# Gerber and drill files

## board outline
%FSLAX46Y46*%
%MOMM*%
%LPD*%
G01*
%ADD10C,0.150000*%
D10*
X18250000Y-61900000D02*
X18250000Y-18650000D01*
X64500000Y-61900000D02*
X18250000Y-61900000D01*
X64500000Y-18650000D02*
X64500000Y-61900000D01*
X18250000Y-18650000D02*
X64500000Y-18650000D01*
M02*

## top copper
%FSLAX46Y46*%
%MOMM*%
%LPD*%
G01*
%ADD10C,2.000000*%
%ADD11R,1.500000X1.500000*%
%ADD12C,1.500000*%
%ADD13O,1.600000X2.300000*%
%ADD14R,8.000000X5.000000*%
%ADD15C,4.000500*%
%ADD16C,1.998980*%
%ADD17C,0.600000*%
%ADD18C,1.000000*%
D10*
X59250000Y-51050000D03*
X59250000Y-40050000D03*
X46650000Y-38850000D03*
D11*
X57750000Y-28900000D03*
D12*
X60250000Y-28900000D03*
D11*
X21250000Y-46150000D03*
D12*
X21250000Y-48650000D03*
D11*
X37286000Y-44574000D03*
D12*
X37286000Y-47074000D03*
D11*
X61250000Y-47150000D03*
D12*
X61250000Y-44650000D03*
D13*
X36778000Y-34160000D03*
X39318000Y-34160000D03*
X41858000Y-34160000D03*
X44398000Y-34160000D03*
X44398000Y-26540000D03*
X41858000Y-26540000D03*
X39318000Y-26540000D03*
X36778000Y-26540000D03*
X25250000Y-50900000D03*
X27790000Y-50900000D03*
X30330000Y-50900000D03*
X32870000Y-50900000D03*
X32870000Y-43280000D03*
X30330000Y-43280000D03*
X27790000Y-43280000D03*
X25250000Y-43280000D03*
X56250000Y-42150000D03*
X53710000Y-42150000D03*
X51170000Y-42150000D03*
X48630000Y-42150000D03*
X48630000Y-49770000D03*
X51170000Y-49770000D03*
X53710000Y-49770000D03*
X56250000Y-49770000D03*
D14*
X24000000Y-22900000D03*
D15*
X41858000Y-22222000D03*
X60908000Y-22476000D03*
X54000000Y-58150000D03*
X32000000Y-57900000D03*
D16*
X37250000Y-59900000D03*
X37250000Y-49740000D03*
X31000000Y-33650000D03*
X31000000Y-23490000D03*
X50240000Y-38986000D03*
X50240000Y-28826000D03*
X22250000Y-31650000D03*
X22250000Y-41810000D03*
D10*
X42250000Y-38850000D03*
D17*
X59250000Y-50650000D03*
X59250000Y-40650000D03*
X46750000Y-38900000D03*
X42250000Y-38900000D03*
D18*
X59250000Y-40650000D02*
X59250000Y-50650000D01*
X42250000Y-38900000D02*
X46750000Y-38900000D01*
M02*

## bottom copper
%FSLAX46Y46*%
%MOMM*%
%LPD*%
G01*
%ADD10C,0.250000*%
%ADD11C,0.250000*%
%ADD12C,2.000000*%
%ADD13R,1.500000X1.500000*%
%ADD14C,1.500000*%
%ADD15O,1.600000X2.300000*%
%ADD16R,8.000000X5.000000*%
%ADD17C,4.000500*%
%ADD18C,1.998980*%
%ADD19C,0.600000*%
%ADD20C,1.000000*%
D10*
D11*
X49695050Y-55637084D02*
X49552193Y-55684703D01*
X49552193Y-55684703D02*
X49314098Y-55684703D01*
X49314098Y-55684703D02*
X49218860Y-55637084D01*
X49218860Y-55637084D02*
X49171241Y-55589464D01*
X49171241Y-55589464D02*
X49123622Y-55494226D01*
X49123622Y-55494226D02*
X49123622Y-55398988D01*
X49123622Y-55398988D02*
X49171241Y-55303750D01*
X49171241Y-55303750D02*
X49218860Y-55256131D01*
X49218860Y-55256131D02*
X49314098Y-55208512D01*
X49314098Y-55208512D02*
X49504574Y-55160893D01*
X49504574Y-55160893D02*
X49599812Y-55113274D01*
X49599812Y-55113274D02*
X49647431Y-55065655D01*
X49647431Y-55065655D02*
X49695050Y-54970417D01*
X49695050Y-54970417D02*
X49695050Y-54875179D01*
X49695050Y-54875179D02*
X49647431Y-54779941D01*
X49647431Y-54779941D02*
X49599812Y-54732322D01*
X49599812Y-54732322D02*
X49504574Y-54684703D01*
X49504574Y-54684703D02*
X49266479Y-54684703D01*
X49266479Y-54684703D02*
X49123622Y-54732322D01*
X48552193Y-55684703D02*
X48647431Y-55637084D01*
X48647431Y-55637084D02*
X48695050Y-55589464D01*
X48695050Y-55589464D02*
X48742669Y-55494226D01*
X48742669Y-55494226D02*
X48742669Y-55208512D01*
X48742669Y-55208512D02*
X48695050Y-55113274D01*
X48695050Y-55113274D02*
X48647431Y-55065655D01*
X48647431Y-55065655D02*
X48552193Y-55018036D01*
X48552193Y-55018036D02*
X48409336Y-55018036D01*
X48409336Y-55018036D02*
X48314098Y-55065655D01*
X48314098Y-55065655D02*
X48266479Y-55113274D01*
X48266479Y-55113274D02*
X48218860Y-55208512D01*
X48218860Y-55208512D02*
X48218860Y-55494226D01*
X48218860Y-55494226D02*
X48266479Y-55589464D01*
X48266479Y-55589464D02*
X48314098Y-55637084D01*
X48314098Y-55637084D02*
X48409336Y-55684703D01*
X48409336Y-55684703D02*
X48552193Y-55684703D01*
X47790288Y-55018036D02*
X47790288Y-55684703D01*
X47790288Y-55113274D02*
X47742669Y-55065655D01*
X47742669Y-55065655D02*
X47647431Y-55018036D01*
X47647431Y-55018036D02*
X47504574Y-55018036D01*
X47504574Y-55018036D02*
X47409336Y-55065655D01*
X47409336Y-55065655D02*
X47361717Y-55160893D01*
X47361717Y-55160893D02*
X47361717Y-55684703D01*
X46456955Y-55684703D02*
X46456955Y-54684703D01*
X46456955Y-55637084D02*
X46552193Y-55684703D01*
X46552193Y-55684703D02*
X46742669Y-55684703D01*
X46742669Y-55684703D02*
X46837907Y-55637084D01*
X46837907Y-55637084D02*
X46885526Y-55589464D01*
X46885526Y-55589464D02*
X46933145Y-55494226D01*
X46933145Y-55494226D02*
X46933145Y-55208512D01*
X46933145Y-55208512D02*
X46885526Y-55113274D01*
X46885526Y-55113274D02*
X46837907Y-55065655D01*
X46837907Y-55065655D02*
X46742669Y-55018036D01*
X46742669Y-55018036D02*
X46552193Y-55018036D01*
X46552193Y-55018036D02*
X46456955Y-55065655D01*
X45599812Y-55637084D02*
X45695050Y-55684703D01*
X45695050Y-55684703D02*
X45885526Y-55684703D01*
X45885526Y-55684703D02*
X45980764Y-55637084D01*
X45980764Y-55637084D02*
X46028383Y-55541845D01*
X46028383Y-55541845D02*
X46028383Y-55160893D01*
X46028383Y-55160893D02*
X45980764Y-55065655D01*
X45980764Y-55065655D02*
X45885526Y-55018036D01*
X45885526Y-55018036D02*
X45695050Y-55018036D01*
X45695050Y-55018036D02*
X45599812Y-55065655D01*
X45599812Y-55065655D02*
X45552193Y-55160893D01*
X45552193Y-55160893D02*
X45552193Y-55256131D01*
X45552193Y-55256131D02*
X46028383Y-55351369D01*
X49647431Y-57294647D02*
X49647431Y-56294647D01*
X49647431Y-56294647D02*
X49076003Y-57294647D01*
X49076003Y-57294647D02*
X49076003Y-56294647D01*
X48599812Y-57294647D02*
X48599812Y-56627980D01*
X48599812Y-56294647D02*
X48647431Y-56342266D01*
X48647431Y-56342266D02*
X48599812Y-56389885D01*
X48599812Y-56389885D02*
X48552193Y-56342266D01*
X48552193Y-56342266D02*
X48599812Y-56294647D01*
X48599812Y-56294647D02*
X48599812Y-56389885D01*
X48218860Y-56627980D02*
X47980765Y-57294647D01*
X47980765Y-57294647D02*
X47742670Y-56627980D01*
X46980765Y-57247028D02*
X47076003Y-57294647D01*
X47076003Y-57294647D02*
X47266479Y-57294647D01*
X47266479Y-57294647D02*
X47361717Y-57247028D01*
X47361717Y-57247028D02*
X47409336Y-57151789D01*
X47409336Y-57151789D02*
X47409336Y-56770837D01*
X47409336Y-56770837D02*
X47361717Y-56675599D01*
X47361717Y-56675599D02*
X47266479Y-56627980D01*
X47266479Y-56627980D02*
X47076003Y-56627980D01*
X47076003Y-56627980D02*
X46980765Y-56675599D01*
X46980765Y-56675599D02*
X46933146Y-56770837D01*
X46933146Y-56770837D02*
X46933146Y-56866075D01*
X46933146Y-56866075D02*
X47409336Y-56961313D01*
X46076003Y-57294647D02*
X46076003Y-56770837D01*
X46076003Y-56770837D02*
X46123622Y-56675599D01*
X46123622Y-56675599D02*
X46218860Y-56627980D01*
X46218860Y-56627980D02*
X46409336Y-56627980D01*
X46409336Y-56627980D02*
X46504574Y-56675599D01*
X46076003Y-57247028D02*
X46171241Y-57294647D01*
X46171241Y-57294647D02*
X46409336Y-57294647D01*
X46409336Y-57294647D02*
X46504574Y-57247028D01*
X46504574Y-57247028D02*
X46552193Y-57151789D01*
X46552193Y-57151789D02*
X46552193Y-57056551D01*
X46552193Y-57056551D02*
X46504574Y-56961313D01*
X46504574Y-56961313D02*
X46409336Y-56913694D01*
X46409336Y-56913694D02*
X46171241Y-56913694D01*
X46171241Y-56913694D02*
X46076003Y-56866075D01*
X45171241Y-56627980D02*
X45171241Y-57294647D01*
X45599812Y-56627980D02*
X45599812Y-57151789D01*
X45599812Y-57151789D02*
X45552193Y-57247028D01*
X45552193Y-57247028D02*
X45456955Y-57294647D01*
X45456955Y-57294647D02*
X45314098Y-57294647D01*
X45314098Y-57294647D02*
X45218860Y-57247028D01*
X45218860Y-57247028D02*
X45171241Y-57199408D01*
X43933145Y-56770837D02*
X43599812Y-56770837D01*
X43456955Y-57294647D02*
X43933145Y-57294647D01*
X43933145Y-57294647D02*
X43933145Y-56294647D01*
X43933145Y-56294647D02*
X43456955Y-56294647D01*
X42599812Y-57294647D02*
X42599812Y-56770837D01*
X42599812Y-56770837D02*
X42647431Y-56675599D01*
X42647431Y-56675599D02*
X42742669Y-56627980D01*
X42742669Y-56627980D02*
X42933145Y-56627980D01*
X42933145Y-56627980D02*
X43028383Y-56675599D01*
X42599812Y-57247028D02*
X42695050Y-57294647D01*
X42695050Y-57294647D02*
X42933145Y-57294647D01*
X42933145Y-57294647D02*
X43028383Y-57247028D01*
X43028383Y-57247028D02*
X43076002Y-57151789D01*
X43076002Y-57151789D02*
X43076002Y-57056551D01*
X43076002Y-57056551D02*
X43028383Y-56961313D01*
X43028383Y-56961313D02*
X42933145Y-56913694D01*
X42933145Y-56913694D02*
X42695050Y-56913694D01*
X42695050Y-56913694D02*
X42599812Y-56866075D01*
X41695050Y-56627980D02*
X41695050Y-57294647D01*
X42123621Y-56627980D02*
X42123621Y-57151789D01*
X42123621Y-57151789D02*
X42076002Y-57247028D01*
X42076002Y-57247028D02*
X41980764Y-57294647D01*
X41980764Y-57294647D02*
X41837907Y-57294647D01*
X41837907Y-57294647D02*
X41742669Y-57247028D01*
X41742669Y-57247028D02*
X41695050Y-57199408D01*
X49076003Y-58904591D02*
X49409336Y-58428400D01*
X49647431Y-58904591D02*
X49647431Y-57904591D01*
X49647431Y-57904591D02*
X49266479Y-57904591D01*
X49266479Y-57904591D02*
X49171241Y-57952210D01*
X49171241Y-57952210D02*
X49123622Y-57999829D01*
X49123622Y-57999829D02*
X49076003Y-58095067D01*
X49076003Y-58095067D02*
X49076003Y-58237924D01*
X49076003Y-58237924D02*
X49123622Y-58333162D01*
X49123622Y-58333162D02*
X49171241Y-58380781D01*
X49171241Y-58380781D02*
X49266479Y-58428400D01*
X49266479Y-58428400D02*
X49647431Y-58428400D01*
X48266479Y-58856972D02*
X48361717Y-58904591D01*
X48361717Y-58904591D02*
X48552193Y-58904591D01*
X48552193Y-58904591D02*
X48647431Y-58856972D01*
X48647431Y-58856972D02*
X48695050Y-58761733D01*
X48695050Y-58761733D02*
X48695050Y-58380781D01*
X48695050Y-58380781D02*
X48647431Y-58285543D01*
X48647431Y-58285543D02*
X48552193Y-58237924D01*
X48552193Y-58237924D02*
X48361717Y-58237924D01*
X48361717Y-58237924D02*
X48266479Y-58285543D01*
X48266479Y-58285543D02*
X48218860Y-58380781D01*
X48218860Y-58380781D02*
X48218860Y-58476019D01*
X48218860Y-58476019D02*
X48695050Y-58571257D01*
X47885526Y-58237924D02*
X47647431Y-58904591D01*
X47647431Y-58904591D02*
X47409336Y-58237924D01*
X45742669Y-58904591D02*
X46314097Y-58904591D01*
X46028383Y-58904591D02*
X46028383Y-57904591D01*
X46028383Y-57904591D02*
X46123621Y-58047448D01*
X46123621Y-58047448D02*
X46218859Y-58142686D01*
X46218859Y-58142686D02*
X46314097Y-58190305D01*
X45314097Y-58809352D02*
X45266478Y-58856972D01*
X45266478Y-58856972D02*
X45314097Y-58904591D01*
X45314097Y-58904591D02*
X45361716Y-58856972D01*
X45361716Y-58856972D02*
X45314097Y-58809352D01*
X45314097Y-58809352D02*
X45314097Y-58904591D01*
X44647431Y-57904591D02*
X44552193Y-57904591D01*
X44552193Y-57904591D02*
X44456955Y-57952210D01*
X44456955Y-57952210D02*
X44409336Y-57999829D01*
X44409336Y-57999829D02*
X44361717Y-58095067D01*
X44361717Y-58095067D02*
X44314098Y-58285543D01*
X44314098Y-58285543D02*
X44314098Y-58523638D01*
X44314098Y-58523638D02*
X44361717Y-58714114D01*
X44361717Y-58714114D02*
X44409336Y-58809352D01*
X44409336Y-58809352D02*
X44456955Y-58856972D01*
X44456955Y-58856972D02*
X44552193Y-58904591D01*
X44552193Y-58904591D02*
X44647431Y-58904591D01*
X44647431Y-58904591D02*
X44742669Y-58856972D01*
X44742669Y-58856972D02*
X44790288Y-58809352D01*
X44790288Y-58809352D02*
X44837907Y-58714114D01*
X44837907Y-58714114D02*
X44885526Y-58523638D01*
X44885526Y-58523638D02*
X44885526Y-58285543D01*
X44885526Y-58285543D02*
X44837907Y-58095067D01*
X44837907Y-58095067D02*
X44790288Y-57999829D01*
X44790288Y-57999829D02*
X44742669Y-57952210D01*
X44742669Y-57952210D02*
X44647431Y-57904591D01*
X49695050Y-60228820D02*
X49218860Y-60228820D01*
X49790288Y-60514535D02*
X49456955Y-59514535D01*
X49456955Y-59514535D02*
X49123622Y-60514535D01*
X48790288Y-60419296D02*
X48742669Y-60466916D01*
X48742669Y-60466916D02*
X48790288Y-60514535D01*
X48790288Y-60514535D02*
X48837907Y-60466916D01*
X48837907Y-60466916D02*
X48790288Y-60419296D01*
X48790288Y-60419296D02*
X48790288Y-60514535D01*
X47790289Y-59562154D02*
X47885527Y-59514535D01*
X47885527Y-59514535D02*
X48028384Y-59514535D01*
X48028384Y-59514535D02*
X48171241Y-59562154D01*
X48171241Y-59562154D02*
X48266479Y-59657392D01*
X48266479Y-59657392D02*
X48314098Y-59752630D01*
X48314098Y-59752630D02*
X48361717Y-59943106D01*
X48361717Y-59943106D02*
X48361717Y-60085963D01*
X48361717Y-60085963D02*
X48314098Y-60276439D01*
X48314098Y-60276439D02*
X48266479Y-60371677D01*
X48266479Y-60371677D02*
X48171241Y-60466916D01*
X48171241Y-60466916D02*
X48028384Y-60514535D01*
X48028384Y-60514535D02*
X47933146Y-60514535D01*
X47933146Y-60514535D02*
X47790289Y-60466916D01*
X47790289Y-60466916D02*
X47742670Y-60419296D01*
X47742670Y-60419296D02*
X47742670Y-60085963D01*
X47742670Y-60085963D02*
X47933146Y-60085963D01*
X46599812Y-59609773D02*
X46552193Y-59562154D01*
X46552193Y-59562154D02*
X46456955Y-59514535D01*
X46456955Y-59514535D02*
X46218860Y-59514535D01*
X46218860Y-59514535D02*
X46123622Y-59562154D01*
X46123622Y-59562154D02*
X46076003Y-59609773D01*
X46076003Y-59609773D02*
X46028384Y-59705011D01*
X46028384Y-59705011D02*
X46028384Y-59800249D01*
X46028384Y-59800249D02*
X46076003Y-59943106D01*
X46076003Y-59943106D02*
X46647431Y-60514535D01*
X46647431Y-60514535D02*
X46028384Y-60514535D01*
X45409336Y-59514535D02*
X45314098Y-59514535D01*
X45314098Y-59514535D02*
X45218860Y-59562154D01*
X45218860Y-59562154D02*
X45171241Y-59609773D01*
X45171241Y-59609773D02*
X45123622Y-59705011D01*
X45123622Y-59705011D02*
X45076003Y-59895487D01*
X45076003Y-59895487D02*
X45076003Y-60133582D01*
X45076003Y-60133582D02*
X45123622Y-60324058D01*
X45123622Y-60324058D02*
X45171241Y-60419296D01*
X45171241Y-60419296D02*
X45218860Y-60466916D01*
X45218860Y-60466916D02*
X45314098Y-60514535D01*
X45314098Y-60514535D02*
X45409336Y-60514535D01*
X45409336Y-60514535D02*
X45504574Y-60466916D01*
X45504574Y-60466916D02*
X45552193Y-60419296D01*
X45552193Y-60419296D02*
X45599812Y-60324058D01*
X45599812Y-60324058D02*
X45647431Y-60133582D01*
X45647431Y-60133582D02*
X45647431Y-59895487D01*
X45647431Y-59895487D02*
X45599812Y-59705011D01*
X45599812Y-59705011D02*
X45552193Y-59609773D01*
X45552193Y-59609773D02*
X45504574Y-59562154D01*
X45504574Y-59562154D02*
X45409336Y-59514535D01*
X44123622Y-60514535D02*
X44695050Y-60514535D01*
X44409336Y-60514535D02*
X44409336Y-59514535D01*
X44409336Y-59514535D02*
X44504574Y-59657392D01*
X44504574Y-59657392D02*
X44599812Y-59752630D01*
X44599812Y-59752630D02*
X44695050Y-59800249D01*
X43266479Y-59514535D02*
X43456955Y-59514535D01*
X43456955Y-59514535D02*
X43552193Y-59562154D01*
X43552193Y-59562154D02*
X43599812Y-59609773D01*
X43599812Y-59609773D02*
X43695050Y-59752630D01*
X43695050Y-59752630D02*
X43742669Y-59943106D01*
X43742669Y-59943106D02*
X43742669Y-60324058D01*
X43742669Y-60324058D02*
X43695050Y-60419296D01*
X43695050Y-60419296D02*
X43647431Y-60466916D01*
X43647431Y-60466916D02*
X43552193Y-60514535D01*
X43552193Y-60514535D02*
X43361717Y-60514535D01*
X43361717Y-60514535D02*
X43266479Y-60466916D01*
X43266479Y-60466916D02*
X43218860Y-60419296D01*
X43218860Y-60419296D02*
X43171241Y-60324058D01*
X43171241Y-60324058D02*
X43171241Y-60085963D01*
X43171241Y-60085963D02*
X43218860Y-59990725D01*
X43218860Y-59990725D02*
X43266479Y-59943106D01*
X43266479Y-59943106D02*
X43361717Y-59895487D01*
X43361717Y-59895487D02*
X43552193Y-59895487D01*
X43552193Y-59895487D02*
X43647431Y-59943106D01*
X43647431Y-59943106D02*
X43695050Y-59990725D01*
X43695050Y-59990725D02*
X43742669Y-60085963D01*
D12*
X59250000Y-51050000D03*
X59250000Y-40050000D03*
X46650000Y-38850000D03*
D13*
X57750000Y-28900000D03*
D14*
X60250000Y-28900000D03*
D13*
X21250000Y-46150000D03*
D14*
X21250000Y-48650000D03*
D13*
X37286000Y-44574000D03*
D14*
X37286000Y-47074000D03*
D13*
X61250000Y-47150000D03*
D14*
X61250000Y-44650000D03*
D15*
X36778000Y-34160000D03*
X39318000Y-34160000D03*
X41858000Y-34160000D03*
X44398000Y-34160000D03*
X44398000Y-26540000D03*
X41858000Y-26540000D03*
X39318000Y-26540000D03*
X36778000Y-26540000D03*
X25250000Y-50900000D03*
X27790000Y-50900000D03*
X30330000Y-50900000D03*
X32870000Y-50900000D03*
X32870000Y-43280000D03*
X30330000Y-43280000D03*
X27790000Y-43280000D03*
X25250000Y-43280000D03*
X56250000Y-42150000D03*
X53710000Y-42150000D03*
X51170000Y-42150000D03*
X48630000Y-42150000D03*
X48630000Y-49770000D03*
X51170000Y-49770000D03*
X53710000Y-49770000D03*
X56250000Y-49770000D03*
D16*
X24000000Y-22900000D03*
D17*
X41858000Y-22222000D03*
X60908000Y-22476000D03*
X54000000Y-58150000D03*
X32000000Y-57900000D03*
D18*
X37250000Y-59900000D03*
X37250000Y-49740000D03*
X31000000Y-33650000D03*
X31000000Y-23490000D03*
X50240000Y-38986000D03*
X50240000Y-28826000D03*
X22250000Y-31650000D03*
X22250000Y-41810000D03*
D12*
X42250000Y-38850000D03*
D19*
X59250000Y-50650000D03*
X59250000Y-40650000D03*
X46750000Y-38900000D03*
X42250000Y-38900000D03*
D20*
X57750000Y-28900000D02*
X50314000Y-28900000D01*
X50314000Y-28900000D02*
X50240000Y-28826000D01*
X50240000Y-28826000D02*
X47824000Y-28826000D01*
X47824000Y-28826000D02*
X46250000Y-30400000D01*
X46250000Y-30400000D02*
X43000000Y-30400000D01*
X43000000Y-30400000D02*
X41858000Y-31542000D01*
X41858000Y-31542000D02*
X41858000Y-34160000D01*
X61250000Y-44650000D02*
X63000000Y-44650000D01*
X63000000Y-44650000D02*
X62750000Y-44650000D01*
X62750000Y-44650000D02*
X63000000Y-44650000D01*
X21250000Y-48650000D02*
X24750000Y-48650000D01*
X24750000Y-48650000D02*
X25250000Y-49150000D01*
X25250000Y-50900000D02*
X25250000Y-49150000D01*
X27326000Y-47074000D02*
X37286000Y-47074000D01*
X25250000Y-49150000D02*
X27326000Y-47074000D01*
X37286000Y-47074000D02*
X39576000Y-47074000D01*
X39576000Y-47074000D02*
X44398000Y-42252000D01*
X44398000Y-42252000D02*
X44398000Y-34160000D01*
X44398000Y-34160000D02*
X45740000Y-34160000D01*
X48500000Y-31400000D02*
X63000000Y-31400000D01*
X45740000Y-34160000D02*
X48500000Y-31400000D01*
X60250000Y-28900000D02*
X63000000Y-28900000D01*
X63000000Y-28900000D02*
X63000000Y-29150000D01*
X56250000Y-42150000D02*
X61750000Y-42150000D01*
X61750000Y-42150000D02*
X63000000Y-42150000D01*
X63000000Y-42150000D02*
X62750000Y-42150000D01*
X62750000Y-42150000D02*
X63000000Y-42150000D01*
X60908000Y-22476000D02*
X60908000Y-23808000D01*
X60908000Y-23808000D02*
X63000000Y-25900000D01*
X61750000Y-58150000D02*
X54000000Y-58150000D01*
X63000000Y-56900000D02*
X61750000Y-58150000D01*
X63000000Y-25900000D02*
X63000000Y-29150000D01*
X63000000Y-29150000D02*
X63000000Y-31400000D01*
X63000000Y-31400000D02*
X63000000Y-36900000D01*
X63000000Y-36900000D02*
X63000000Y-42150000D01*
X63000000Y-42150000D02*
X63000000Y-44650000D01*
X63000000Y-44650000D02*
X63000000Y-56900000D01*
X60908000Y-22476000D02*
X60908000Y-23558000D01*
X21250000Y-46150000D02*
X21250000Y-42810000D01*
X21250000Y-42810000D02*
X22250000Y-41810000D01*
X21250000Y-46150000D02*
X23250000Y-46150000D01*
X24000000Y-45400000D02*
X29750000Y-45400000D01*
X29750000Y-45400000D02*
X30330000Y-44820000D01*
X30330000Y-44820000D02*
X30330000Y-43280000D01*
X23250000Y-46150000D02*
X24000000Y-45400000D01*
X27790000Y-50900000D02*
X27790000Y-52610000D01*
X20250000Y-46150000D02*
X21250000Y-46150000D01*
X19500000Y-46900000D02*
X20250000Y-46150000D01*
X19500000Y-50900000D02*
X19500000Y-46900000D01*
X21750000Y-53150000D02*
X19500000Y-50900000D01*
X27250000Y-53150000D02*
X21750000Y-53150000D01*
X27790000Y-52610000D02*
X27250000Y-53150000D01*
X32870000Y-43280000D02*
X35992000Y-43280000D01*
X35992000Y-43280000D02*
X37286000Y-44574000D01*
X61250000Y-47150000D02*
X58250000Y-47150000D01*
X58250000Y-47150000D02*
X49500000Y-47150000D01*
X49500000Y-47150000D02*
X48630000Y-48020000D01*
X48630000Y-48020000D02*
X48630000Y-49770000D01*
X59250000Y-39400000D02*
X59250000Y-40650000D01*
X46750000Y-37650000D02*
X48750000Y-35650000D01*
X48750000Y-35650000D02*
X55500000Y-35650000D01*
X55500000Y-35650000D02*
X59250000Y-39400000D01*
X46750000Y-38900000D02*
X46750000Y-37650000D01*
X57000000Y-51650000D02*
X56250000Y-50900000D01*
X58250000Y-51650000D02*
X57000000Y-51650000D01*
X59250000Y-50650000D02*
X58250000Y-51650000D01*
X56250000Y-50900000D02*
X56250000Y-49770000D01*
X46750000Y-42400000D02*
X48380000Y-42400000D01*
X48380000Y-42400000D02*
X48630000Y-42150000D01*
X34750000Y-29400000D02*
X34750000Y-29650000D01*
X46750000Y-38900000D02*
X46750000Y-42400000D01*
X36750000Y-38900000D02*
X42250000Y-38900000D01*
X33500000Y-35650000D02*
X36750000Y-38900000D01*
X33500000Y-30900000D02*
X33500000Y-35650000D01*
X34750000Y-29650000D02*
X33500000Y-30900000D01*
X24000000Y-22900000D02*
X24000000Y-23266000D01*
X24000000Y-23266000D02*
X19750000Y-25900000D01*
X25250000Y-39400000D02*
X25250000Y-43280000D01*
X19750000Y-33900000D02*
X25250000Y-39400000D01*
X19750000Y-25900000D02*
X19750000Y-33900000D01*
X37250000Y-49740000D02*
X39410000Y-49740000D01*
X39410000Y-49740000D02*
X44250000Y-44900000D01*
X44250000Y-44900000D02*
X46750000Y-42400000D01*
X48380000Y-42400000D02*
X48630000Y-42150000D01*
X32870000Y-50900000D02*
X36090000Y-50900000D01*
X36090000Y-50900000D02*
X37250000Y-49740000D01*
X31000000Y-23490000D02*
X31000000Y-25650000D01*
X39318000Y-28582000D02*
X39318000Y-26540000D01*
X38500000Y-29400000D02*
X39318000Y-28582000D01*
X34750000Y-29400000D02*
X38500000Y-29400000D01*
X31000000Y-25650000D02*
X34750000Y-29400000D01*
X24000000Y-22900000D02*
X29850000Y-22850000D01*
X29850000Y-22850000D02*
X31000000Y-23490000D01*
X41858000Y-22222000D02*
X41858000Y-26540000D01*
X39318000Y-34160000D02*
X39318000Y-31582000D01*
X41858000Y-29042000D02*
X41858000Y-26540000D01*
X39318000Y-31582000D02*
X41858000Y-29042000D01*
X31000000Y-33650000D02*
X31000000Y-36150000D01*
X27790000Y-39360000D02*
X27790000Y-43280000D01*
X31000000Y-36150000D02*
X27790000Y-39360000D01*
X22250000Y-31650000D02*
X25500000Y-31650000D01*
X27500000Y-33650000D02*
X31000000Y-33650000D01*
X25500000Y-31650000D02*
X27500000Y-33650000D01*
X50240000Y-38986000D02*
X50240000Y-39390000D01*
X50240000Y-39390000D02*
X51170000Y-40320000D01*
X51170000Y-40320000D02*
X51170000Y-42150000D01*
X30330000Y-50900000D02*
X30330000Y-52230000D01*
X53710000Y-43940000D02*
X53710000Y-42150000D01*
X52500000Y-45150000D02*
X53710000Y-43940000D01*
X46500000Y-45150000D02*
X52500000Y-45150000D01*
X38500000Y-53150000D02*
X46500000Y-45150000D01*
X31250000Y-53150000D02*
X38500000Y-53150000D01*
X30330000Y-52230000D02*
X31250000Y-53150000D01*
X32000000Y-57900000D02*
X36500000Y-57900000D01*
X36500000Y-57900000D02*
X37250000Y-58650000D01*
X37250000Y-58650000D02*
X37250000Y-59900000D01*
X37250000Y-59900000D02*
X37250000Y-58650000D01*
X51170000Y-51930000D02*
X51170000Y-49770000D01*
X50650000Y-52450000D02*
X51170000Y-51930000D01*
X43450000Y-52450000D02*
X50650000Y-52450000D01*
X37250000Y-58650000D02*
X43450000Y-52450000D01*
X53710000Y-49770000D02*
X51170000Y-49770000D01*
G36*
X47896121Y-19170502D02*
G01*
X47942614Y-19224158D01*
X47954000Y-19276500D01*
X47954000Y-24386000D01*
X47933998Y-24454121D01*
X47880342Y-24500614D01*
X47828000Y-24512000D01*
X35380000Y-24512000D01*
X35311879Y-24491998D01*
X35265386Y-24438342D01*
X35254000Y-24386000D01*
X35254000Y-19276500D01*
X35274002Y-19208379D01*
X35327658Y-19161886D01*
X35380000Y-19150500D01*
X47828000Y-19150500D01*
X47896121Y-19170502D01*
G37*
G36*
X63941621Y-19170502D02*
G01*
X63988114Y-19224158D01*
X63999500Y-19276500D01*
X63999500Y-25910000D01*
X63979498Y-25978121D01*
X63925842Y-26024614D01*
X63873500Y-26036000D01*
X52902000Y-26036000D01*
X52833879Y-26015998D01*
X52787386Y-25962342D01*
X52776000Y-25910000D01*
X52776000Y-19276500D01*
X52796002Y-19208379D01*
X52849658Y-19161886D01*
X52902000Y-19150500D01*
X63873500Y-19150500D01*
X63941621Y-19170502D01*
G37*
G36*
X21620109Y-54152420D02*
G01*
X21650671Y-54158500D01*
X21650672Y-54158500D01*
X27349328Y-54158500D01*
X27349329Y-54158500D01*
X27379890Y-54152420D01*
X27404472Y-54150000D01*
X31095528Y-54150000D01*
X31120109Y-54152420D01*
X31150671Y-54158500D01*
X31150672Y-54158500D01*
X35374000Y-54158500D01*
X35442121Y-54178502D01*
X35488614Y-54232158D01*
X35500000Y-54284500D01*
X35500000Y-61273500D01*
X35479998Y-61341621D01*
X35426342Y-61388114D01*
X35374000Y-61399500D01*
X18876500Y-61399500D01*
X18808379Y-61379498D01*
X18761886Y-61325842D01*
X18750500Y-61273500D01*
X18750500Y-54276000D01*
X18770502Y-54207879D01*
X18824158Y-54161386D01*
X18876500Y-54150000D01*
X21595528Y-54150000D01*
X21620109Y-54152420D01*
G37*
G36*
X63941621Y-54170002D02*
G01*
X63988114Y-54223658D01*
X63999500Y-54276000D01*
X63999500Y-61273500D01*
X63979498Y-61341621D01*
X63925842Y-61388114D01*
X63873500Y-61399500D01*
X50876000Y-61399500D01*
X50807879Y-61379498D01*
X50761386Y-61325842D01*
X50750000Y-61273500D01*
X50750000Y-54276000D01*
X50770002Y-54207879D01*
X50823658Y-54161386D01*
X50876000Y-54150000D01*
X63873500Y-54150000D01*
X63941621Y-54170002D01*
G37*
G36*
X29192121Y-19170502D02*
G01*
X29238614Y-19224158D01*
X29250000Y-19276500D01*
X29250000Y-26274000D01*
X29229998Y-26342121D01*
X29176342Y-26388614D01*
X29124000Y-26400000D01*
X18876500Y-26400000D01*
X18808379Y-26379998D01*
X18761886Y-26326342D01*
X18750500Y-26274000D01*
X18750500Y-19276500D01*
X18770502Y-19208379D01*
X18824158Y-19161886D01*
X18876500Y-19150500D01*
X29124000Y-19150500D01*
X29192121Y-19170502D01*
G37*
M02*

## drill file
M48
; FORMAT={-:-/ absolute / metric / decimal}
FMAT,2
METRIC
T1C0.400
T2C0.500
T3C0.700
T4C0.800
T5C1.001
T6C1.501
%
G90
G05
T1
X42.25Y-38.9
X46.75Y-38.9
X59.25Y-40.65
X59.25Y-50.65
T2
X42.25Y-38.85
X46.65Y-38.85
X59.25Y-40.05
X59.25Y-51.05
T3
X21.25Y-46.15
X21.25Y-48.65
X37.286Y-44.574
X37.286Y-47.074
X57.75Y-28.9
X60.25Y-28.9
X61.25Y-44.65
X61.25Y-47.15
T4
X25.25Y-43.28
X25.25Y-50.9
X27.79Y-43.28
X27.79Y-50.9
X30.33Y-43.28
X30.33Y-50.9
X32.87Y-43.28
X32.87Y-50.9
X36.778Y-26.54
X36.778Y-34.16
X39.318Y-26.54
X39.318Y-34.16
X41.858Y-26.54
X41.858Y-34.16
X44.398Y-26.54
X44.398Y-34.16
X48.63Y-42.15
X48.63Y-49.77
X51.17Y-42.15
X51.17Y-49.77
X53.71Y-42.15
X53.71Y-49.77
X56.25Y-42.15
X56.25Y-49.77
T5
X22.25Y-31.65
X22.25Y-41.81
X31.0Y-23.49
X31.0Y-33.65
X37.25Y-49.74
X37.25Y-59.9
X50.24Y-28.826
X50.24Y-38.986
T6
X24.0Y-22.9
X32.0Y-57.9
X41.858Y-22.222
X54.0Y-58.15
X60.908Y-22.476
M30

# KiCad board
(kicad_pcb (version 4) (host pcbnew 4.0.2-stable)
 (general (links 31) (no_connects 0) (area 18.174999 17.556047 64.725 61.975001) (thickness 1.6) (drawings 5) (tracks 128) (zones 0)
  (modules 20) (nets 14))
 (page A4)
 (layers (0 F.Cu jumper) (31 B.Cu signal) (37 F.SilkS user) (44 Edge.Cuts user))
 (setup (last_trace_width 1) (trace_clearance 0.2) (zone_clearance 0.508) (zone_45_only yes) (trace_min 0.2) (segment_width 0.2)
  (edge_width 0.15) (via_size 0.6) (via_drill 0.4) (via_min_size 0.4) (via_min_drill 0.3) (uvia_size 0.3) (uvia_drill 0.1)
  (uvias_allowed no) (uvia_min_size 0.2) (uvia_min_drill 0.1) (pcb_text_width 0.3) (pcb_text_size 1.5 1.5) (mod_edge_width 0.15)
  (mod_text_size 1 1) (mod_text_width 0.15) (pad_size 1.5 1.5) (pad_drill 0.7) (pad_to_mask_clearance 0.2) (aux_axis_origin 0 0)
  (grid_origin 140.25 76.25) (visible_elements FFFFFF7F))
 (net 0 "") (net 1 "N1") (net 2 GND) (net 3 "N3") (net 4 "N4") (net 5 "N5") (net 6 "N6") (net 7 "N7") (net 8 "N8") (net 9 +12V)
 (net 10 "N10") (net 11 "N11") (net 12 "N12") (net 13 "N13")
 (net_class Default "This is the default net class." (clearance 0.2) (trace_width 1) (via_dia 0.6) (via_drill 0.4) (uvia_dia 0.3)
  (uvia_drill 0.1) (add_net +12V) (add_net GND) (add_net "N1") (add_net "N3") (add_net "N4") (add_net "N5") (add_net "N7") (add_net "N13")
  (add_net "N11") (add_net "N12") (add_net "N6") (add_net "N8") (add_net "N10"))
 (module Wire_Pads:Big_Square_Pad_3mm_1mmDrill (layer F.Cu) (at 59.25 51.05)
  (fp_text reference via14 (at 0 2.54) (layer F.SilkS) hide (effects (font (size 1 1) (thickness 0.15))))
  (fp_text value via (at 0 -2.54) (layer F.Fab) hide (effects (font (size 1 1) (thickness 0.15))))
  (pad 1 thru_hole circle (at 0 0) (size 2 2) (drill 0.5) (layers *.Cu *.Mask F.SilkS)))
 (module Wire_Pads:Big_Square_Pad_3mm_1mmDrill (layer F.Cu) (at 59.25 40.05)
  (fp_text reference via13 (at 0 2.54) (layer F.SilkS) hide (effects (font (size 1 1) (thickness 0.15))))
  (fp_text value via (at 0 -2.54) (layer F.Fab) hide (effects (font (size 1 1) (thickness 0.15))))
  (pad 1 thru_hole circle (at 0 0) (size 2 2) (drill 0.5) (layers *.Cu *.Mask F.SilkS)))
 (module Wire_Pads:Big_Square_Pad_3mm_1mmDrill (layer F.Cu) (at 46.65 38.85)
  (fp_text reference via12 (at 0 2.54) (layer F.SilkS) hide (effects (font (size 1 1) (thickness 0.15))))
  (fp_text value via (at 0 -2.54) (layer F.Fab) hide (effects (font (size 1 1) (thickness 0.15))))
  (pad 1 thru_hole circle (at 0 0) (size 2 2) (drill 0.5) (layers *.Cu *.Mask F.SilkS)))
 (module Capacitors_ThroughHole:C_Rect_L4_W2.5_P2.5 (layer F.Cu) (at 57.75 28.9)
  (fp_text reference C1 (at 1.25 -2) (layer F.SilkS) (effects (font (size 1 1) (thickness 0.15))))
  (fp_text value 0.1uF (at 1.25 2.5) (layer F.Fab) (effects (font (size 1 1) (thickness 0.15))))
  (pad 1 thru_hole rect (at 0 0) (size 1.5 1.5) (drill 0.7) (layers *.Cu *.Mask F.SilkS) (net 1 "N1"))
  (pad 2 thru_hole circle (at 2.5 0) (size 1.5 1.5) (drill 0.7) (layers *.Cu *.Mask F.SilkS) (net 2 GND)))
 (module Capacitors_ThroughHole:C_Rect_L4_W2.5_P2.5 (layer F.Cu) (at 21.25 46.15 270)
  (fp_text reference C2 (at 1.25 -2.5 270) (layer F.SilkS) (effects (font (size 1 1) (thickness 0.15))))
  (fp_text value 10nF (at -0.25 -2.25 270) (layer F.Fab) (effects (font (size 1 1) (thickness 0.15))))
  (pad 1 thru_hole rect (at 0 0 270) (size 1.5 1.5) (drill 0.7) (layers *.Cu *.Mask F.SilkS) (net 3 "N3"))
  (pad 2 thru_hole circle (at 2.5 0 270) (size 1.5 1.5) (drill 0.7) (layers *.Cu *.Mask F.SilkS) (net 2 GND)))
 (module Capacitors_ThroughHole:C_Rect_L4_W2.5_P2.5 (layer F.Cu) (at 37.286 44.574 270)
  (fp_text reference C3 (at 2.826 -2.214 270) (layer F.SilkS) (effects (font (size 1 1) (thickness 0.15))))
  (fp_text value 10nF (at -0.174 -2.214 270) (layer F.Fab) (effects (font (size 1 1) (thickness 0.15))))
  (pad 1 thru_hole rect (at 0 0 270) (size 1.5 1.5) (drill 0.7) (layers *.Cu *.Mask F.SilkS) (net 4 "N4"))
  (pad 2 thru_hole circle (at 2.5 0 270) (size 1.5 1.5) (drill 0.7) (layers *.Cu *.Mask F.SilkS) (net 2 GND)))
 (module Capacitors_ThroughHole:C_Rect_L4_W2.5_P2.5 (layer F.Cu) (at 61.25 47.15 90)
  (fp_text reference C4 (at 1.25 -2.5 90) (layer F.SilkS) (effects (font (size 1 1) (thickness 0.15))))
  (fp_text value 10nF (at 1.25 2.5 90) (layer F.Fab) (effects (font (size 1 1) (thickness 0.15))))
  (pad 1 thru_hole rect (at 0 0 90) (size 1.5 1.5) (drill 0.7) (layers *.Cu *.Mask F.SilkS) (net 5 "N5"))
  (pad 2 thru_hole circle (at 2.5 0 90) (size 1.5 1.5) (drill 0.7) (layers *.Cu *.Mask F.SilkS) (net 2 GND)))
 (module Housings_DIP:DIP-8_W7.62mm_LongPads (layer F.Cu) (at 36.778 34.16 90)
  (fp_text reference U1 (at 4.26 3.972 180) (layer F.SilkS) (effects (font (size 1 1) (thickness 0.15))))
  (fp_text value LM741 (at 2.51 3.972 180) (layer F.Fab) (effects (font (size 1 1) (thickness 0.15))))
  (pad 1 thru_hole oval (at 0 0 90) (size 2.3 1.6) (drill 0.8) (layers *.Cu *.Mask F.SilkS) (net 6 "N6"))
  (pad 2 thru_hole oval (at 0 2.54 90) (size 2.3 1.6) (drill 0.8) (layers *.Cu *.Mask F.SilkS) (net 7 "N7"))
  (pad 3 thru_hole oval (at 0 5.08 90) (size 2.3 1.6) (drill 0.8) (layers *.Cu *.Mask F.SilkS) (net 1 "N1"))
  (pad 4 thru_hole oval (at 0 7.62 90) (size 2.3 1.6) (drill 0.8) (layers *.Cu *.Mask F.SilkS) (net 2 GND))
  (pad 5 thru_hole oval (at 7.62 7.62 90) (size 2.3 1.6) (drill 0.8) (layers *.Cu *.Mask F.SilkS) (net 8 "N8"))
  (pad 6 thru_hole oval (at 7.62 5.08 90) (size 2.3 1.6) (drill 0.8) (layers *.Cu *.Mask F.SilkS) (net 7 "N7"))
  (pad 7 thru_hole oval (at 7.62 2.54 90) (size 2.3 1.6) (drill 0.8) (layers *.Cu *.Mask F.SilkS) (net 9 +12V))
  (pad 8 thru_hole oval (at 7.62 0 90) (size 2.3 1.6) (drill 0.8) (layers *.Cu *.Mask F.SilkS)))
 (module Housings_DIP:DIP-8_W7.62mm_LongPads (layer F.Cu) (at 25.25 50.9 90)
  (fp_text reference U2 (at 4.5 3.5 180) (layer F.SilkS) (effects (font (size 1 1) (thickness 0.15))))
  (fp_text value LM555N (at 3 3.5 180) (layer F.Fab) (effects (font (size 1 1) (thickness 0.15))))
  (pad 1 thru_hole oval (at 0 0 90) (size 2.3 1.6) (drill 0.8) (layers *.Cu *.Mask F.SilkS) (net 2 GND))
  (pad 2 thru_hole oval (at 0 2.54 90) (size 2.3 1.6) (drill 0.8) (layers *.Cu *.Mask F.SilkS) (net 3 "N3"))
  (pad 3 thru_hole oval (at 0 5.08 90) (size 2.3 1.6) (drill 0.8) (layers *.Cu *.Mask F.SilkS) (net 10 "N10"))
  (pad 4 thru_hole oval (at 0 7.62 90) (size 2.3 1.6) (drill 0.8) (layers *.Cu *.Mask F.SilkS) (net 9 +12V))
  (pad 5 thru_hole oval (at 7.62 7.62 90) (size 2.3 1.6) (drill 0.8) (layers *.Cu *.Mask F.SilkS) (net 4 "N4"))
  (pad 6 thru_hole oval (at 7.62 5.08 90) (size 2.3 1.6) (drill 0.8) (layers *.Cu *.Mask F.SilkS) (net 3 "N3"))
  (pad 7 thru_hole oval (at 7.62 2.54 90) (size 2.3 1.6) (drill 0.8) (layers *.Cu *.Mask F.SilkS) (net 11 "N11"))
  (pad 8 thru_hole oval (at 7.62 0 90) (size 2.3 1.6) (drill 0.8) (layers *.Cu *.Mask F.SilkS) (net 9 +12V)))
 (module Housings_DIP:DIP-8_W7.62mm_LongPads (layer F.Cu) (at 56.25 42.15 270)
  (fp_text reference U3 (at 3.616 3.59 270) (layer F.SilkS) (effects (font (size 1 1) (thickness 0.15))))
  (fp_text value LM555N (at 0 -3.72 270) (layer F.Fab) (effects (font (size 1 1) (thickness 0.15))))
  (pad 1 thru_hole oval (at 0 0 270) (size 2.3 1.6) (drill 0.8) (layers *.Cu *.Mask F.SilkS) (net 2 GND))
  (pad 2 thru_hole oval (at 0 2.54 270) (size 2.3 1.6) (drill 0.8) (layers *.Cu *.Mask F.SilkS) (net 10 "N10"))
  (pad 3 thru_hole oval (at 0 5.08 270) (size 2.3 1.6) (drill 0.8) (layers *.Cu *.Mask F.SilkS) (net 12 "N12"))
  (pad 4 thru_hole oval (at 0 7.62 270) (size 2.3 1.6) (drill 0.8) (layers *.Cu *.Mask F.SilkS) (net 9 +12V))
  (pad 5 thru_hole oval (at 7.62 7.62 270) (size 2.3 1.6) (drill 0.8) (layers *.Cu *.Mask F.SilkS) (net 5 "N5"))
  (pad 6 thru_hole oval (at 7.62 5.08 270) (size 2.3 1.6) (drill 0.8) (layers *.Cu *.Mask F.SilkS) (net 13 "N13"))
  (pad 7 thru_hole oval (at 7.62 2.54 270) (size 2.3 1.6) (drill 0.8) (layers *.Cu *.Mask F.SilkS) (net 13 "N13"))
  (pad 8 thru_hole oval (at 7.62 0 270) (size 2.3 1.6) (drill 0.8) (layers *.Cu *.Mask F.SilkS) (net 9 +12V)))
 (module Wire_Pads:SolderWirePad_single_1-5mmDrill (layer F.Cu) (at 24 22.9 180)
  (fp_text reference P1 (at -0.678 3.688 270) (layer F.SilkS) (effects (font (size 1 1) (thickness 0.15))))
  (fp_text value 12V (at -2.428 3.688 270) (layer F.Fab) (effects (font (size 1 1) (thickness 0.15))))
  (pad 1 thru_hole rect (at 0 0 180) (size 8 5) (drill 1.50114) (layers *.Cu *.Mask F.SilkS) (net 9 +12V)))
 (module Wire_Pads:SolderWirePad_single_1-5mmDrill (layer F.Cu) (at 41.858 22.222 270)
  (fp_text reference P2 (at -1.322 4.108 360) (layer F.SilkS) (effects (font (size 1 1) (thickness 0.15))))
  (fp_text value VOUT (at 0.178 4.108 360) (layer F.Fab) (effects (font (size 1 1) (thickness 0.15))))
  (pad 1 thru_hole circle (at 0 0 270) (size 4.0005 4.0005) (drill 1.50114) (layers *.Cu *.Mask F.SilkS) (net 7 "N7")))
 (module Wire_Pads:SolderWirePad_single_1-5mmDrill (layer F.Cu) (at 60.908 22.476)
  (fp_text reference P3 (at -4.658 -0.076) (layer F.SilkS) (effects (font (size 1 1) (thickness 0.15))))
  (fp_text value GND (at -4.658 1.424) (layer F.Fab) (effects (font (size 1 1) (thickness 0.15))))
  (pad 1 thru_hole circle (at 0 0) (size 4.0005 4.0005) (drill 1.50114) (layers *.Cu *.Mask F.SilkS) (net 2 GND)))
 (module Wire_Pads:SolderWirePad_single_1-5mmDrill (layer F.Cu) (at 54 58.15)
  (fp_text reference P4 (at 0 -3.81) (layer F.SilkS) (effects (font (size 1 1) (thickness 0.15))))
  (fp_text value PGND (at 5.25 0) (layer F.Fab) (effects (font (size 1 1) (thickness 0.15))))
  (pad 1 thru_hole circle (at 0 0) (size 4.0005 4.0005) (drill 1.50114) (layers *.Cu *.Mask F.SilkS) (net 2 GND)))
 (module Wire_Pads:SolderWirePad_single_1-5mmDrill (layer F.Cu) (at 32 57.9)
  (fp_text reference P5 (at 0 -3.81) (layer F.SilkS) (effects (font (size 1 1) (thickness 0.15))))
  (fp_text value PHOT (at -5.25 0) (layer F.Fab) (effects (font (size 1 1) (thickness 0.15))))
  (pad 1 thru_hole circle (at 0 0) (size 4.0005 4.0005) (drill 1.50114) (layers *.Cu *.Mask F.SilkS) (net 13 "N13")))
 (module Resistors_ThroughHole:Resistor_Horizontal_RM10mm (layer F.Cu) (at 37.25 59.9 90)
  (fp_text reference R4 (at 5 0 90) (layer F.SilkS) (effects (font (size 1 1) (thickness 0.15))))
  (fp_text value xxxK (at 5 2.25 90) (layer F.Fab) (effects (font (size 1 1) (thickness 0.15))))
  (pad 1 thru_hole circle (at 0 0 90) (size 1.99898 1.99898) (drill 1.00076) (layers *.Cu *.SilkS *.Mask) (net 13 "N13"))
  (pad 2 thru_hole circle (at 10.16 0 90) (size 1.99898 1.99898) (drill 1.00076) (layers *.Cu *.SilkS *.Mask) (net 9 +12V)))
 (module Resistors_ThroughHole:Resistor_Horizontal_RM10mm (layer F.Cu) (at 31 33.65 90)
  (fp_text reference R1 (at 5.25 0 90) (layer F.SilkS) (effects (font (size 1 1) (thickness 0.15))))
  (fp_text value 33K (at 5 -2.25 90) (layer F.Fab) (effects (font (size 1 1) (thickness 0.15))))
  (pad 1 thru_hole circle (at 0 0 90) (size 1.99898 1.99898) (drill 1.00076) (layers *.Cu *.SilkS *.Mask) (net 11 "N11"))
  (pad 2 thru_hole circle (at 10.16 0 90) (size 1.99898 1.99898) (drill 1.00076) (layers *.Cu *.SilkS *.Mask) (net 9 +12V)))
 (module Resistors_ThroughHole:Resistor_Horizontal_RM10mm (layer F.Cu) (at 50.24 38.986 90)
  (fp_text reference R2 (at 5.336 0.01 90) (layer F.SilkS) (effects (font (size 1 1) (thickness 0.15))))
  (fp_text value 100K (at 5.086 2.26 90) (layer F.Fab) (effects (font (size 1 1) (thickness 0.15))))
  (pad 1 thru_hole circle (at 0 0 90) (size 1.99898 1.99898) (drill 1.00076) (layers *.Cu *.SilkS *.Mask) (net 12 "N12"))
  (pad 2 thru_hole circle (at 10.16 0 90) (size 1.99898 1.99898) (drill 1.00076) (layers *.Cu *.SilkS *.Mask) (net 1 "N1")))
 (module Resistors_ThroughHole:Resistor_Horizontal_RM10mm (layer F.Cu) (at 22.25 31.65 270)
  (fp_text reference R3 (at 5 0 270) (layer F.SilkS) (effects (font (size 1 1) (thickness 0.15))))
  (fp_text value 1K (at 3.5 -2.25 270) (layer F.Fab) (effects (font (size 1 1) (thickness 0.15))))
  (pad 1 thru_hole circle (at 0 0 270) (size 1.99898 1.99898) (drill 1.00076) (layers *.Cu *.SilkS *.Mask) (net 11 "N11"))
  (pad 2 thru_hole circle (at 10.16 0 270) (size 1.99898 1.99898) (drill 1.00076) (layers *.Cu *.SilkS *.Mask) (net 3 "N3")))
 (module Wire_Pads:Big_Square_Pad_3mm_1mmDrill (layer F.Cu) (at 42.25 38.85)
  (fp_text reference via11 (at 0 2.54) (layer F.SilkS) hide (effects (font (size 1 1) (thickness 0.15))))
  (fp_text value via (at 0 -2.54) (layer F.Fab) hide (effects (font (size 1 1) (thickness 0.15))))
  (pad 1 thru_hole circle (at 0 0) (size 2 2) (drill 0.5) (layers *.Cu *.Mask F.SilkS)))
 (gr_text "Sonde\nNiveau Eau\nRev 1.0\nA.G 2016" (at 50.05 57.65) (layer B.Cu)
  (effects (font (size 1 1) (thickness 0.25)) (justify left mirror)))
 (gr_line (start 18.25 61.9) (end 18.25 18.65) (angle 90) (layer Edge.Cuts) (width 0.15))
 (gr_line (start 64.5 61.9) (end 18.25 61.9) (angle 90) (layer Edge.Cuts) (width 0.15))
 (gr_line (start 64.5 18.65) (end 64.5 61.9) (angle 90) (layer Edge.Cuts) (width 0.15))
 (gr_line (start 18.25 18.65) (end 64.5 18.65) (angle 90) (layer Edge.Cuts) (width 0.15))
 (segment (start 57.75 28.9) (end 50.314 28.9) (width 1) (layer B.Cu) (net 1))
 (segment (start 50.314 28.9) (end 50.24 28.826) (width 1) (layer B.Cu) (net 1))
 (segment (start 50.24 28.826) (end 47.824 28.826) (width 1) (layer B.Cu) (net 1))
 (segment (start 47.824 28.826) (end 46.25 30.4) (width 1) (layer B.Cu) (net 1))
 (segment (start 46.25 30.4) (end 43 30.4) (width 1) (layer B.Cu) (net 1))
 (segment (start 43 30.4) (end 41.858 31.542) (width 1) (layer B.Cu) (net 1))
 (segment (start 41.858 31.542) (end 41.858 34.16) (width 1) (layer B.Cu) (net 1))
 (segment (start 61.25 44.65) (end 63 44.65) (width 1) (layer B.Cu) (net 2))
 (segment (start 63 44.65) (end 62.75 44.65) (width 1) (layer B.Cu) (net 2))
 (segment (start 62.75 44.65) (end 63 44.65) (width 1) (layer B.Cu) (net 2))
 (segment (start 21.25 48.65) (end 24.75 48.65) (width 1) (layer B.Cu) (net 2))
 (segment (start 24.75 48.65) (end 25.25 49.15) (width 1) (layer B.Cu) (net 2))
 (segment (start 25.25 50.9) (end 25.25 49.15) (width 1) (layer B.Cu) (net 2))
 (segment (start 27.326 47.074) (end 37.286 47.074) (width 1) (layer B.Cu) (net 2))
 (segment (start 25.25 49.15) (end 27.326 47.074) (width 1) (layer B.Cu) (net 2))
 (segment (start 37.286 47.074) (end 39.576 47.074) (width 1) (layer B.Cu) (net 2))
 (segment (start 39.576 47.074) (end 44.398 42.252) (width 1) (layer B.Cu) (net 2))
 (segment (start 44.398 42.252) (end 44.398 34.16) (width 1) (layer B.Cu) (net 2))
 (segment (start 44.398 34.16) (end 45.74 34.16) (width 1) (layer B.Cu) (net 2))
 (segment (start 48.5 31.4) (end 63 31.4) (width 1) (layer B.Cu) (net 2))
 (segment (start 45.74 34.16) (end 48.5 31.4) (width 1) (layer B.Cu) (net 2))
 (segment (start 60.25 28.9) (end 63 28.9) (width 1) (layer B.Cu) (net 2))
 (segment (start 63 28.9) (end 63 29.15) (width 1) (layer B.Cu) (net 2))
 (segment (start 56.25 42.15) (end 61.75 42.15) (width 1) (layer B.Cu) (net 2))
 (segment (start 61.75 42.15) (end 63 42.15) (width 1) (layer B.Cu) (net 2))
 (segment (start 63 42.15) (end 62.75 42.15) (width 1) (layer B.Cu) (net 2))
 (segment (start 62.75 42.15) (end 63 42.15) (width 1) (layer B.Cu) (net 2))
 (segment (start 60.908 22.476) (end 60.908 23.808) (width 1) (layer B.Cu) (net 2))
 (segment (start 60.908 23.808) (end 63 25.9) (width 1) (layer B.Cu) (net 2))
 (segment (start 61.75 58.15) (end 54 58.15) (width 1) (layer B.Cu) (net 2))
 (segment (start 63 56.9) (end 61.75 58.15) (width 1) (layer B.Cu) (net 2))
 (segment (start 63 25.9) (end 63 29.15) (width 1) (layer B.Cu) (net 2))
 (segment (start 63 29.15) (end 63 31.4) (width 1) (layer B.Cu) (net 2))
 (segment (start 63 31.4) (end 63 36.9) (width 1) (layer B.Cu) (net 2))
 (segment (start 63 36.9) (end 63 42.15) (width 1) (layer B.Cu) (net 2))
 (segment (start 63 42.15) (end 63 44.65) (width 1) (layer B.Cu) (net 2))
 (segment (start 63 44.65) (end 63 56.9) (width 1) (layer B.Cu) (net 2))
 (segment (start 60.908 22.476) (end 60.908 23.558) (width 1) (layer B.Cu) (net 2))
 (segment (start 21.25 46.15) (end 21.25 42.81) (width 1) (layer B.Cu) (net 3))
 (segment (start 21.25 42.81) (end 22.25 41.81) (width 1) (layer B.Cu) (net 3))
 (segment (start 21.25 46.15) (end 23.25 46.15) (width 1) (layer B.Cu) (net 3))
 (segment (start 24 45.4) (end 29.75 45.4) (width 1) (layer B.Cu) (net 3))
 (segment (start 29.75 45.4) (end 30.33 44.82) (width 1) (layer B.Cu) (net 3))
 (segment (start 30.33 44.82) (end 30.33 43.28) (width 1) (layer B.Cu) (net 3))
 (segment (start 23.25 46.15) (end 24 45.4) (width 1) (layer B.Cu) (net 3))
 (segment (start 27.79 50.9) (end 27.79 52.61) (width 1) (layer B.Cu) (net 3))
 (segment (start 20.25 46.15) (end 21.25 46.15) (width 1) (layer B.Cu) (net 3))
 (segment (start 19.5 46.9) (end 20.25 46.15) (width 1) (layer B.Cu) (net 3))
 (segment (start 19.5 50.9) (end 19.5 46.9) (width 1) (layer B.Cu) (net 3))
 (segment (start 21.75 53.15) (end 19.5 50.9) (width 1) (layer B.Cu) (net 3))
 (segment (start 27.25 53.15) (end 21.75 53.15) (width 1) (layer B.Cu) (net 3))
 (segment (start 27.79 52.61) (end 27.25 53.15) (width 1) (layer B.Cu) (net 3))
 (segment (start 32.87 43.28) (end 35.992 43.28) (width 1) (layer B.Cu) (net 4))
 (segment (start 35.992 43.28) (end 37.286 44.574) (width 1) (layer B.Cu) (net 4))
 (segment (start 61.25 47.15) (end 58.25 47.15) (width 1) (layer B.Cu) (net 5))
 (segment (start 58.25 47.15) (end 49.5 47.15) (width 1) (layer B.Cu) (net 5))
 (segment (start 49.5 47.15) (end 48.63 48.02) (width 1) (layer B.Cu) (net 5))
 (segment (start 48.63 48.02) (end 48.63 49.77) (width 1) (layer B.Cu) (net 5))
 (segment (start 59.25 39.4) (end 59.25 40.65) (width 1) (layer B.Cu) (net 9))
 (segment (start 46.75 37.65) (end 48.75 35.65) (width 1) (layer B.Cu) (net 9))
 (segment (start 48.75 35.65) (end 55.5 35.65) (width 1) (layer B.Cu) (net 9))
 (segment (start 55.5 35.65) (end 59.25 39.4) (width 1) (layer B.Cu) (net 9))
 (segment (start 46.75 38.9) (end 46.75 37.65) (width 1) (layer B.Cu) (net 9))
 (segment (start 57 51.65) (end 56.25 50.9) (width 1) (layer B.Cu) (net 9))
 (segment (start 58.25 51.65) (end 57 51.65) (width 1) (layer B.Cu) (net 9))
 (segment (start 59.25 50.65) (end 58.25 51.65) (width 1) (layer B.Cu) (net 9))
 (via (at 59.25 50.65) (size 0.6) (drill 0.4) (layers F.Cu B.Cu) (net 9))
 (segment (start 59.25 40.65) (end 59.25 50.65) (width 1) (layer F.Cu) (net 9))
 (via (at 59.25 40.65) (size 0.6) (drill 0.4) (layers F.Cu B.Cu) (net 9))
 (segment (start 56.25 50.9) (end 56.25 49.77) (width 1) (layer B.Cu) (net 9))
 (segment (start 46.75 42.4) (end 48.38 42.4) (width 1) (layer B.Cu) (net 9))
 (segment (start 48.38 42.4) (end 48.63 42.15) (width 1) (layer B.Cu) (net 9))
 (segment (start 34.75 29.4) (end 34.75 29.65) (width 1) (layer B.Cu) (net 9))
 (segment (start 46.75 38.9) (end 46.75 42.4) (width 1) (layer B.Cu) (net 9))
 (via (at 46.75 38.9) (size 0.6) (drill 0.4) (layers F.Cu B.Cu) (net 9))
 (segment (start 42.25 38.9) (end 46.75 38.9) (width 1) (layer F.Cu) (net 9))
 (via (at 42.25 38.9) (size 0.6) (drill 0.4) (layers F.Cu B.Cu) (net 9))
 (segment (start 36.75 38.9) (end 42.25 38.9) (width 1) (layer B.Cu) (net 9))
 (segment (start 33.5 35.65) (end 36.75 38.9) (width 1) (layer B.Cu) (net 9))
 (segment (start 33.5 30.9) (end 33.5 35.65) (width 1) (layer B.Cu) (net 9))
 (segment (start 34.75 29.65) (end 33.5 30.9) (width 1) (layer B.Cu) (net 9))
 (segment (start 24 22.9) (end 24 23.266) (width 1) (layer B.Cu) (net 9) (status 30))
 (segment (start 24 23.266) (end 19.75 25.9) (width 1) (layer B.Cu) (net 9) (status 10))
 (segment (start 25.25 39.4) (end 25.25 43.28) (width 1) (layer B.Cu) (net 9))
 (segment (start 19.75 33.9) (end 25.25 39.4) (width 1) (layer B.Cu) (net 9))
 (segment (start 19.75 25.9) (end 19.75 33.9) (width 1) (layer B.Cu) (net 9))
 (segment (start 37.25 49.74) (end 39.41 49.74) (width 1) (layer B.Cu) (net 9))
 (segment (start 39.41 49.74) (end 44.25 44.9) (width 1) (layer B.Cu) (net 9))
 (segment (start 44.25 44.9) (end 46.75 42.4) (width 1) (layer B.Cu) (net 9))
 (segment (start 48.38 42.4) (end 48.63 42.15) (width 1) (layer B.Cu) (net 9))
 (segment (start 32.87 50.9) (end 36.09 50.9) (width 1) (layer B.Cu) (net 9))
 (segment (start 36.09 50.9) (end 37.25 49.74) (width 1) (layer B.Cu) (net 9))
 (segment (start 31 23.49) (end 31 25.65) (width 1) (layer B.Cu) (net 9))
 (segment (start 39.318 28.582) (end 39.318 26.54) (width 1) (layer B.Cu) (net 9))
 (segment (start 38.5 29.4) (end 39.318 28.582) (width 1) (layer B.Cu) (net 9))
 (segment (start 34.75 29.4) (end 38.5 29.4) (width 1) (layer B.Cu) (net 9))
 (segment (start 31 25.65) (end 34.75 29.4) (width 1) (layer B.Cu) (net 9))
 (segment (start 24 22.9) (end 29.85 22.85) (width 1) (layer B.Cu) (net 9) (status 10))
 (segment (start 29.85 22.85) (end 31 23.49) (width 1) (layer B.Cu) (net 9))
 (segment (start 41.858 22.222) (end 41.858 26.54) (width 1) (layer B.Cu) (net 7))
 (segment (start 39.318 34.16) (end 39.318 31.582) (width 1) (layer B.Cu) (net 7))
 (segment (start 41.858 29.042) (end 41.858 26.54) (width 1) (layer B.Cu) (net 7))
 (segment (start 39.318 31.582) (end 41.858 29.042) (width 1) (layer B.Cu) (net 7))
 (segment (start 31 33.65) (end 31 36.15) (width 1) (layer B.Cu) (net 11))
 (segment (start 27.79 39.36) (end 27.79 43.28) (width 1) (layer B.Cu) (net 11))
 (segment (start 31 36.15) (end 27.79 39.36) (width 1) (layer B.Cu) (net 11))
 (segment (start 22.25 31.65) (end 25.5 31.65) (width 1) (layer B.Cu) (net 11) (status 10))
 (segment (start 27.5 33.65) (end 31 33.65) (width 1) (layer B.Cu) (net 11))
 (segment (start 25.5 31.65) (end 27.5 33.65) (width 1) (layer B.Cu) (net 11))
 (segment (start 50.24 38.986) (end 50.24 39.39) (width 1) (layer B.Cu) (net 12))
 (segment (start 50.24 39.39) (end 51.17 40.32) (width 1) (layer B.Cu) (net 12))
 (segment (start 51.17 40.32) (end 51.17 42.15) (width 1) (layer B.Cu) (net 12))
 (segment (start 30.33 50.9) (end 30.33 52.23) (width 1) (layer B.Cu) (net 10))
 (segment (start 53.71 43.94) (end 53.71 42.15) (width 1) (layer B.Cu) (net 10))
 (segment (start 52.5 45.15) (end 53.71 43.94) (width 1) (layer B.Cu) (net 10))
 (segment (start 46.5 45.15) (end 52.5 45.15) (width 1) (layer B.Cu) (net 10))
 (segment (start 38.5 53.15) (end 46.5 45.15) (width 1) (layer B.Cu) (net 10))
 (segment (start 31.25 53.15) (end 38.5 53.15) (width 1) (layer B.Cu) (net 10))
 (segment (start 30.33 52.23) (end 31.25 53.15) (width 1) (layer B.Cu) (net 10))
 (segment (start 32 57.9) (end 36.5 57.9) (width 1) (layer B.Cu) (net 13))
 (segment (start 36.5 57.9) (end 37.25 58.65) (width 1) (layer B.Cu) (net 13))
 (segment (start 37.25 58.65) (end 37.25 59.9) (width 1) (layer B.Cu) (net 13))
 (segment (start 37.25 59.9) (end 37.25 58.65) (width 1) (layer B.Cu) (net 13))
 (segment (start 51.17 51.93) (end 51.17 49.77) (width 1) (layer B.Cu) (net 13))
 (segment (start 50.65 52.45) (end 51.17 51.93) (width 1) (layer B.Cu) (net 13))
 (segment (start 43.45 52.45) (end 50.65 52.45) (width 1) (layer B.Cu) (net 13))
 (segment (start 37.25 58.65) (end 43.45 52.45) (width 1) (layer B.Cu) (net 13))
 (segment (start 53.71 49.77) (end 51.17 49.77) (width 1) (layer B.Cu) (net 13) (status 30))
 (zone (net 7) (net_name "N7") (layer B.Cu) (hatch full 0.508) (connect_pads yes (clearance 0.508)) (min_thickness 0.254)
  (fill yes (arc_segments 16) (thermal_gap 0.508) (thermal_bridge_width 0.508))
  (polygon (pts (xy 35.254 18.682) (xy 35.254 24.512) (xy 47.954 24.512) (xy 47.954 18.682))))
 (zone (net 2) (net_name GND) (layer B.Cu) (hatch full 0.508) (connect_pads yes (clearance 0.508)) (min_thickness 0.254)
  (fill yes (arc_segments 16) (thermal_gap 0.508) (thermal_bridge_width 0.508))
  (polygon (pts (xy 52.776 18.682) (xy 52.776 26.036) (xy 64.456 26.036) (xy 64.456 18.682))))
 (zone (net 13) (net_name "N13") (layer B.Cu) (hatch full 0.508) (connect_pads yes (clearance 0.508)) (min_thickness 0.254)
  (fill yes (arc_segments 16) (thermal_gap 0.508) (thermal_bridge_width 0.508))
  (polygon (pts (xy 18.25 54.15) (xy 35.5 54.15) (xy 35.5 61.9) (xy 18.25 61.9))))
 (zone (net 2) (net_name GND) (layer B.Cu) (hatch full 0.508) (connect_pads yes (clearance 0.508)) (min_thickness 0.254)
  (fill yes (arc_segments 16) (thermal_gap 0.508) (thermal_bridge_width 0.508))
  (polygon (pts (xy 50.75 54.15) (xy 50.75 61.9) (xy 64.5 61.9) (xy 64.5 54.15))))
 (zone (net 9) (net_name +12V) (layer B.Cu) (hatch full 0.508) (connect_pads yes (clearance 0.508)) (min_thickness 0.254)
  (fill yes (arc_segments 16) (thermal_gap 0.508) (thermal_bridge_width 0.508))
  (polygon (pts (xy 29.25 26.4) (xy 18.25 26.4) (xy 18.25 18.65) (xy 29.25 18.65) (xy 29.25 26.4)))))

